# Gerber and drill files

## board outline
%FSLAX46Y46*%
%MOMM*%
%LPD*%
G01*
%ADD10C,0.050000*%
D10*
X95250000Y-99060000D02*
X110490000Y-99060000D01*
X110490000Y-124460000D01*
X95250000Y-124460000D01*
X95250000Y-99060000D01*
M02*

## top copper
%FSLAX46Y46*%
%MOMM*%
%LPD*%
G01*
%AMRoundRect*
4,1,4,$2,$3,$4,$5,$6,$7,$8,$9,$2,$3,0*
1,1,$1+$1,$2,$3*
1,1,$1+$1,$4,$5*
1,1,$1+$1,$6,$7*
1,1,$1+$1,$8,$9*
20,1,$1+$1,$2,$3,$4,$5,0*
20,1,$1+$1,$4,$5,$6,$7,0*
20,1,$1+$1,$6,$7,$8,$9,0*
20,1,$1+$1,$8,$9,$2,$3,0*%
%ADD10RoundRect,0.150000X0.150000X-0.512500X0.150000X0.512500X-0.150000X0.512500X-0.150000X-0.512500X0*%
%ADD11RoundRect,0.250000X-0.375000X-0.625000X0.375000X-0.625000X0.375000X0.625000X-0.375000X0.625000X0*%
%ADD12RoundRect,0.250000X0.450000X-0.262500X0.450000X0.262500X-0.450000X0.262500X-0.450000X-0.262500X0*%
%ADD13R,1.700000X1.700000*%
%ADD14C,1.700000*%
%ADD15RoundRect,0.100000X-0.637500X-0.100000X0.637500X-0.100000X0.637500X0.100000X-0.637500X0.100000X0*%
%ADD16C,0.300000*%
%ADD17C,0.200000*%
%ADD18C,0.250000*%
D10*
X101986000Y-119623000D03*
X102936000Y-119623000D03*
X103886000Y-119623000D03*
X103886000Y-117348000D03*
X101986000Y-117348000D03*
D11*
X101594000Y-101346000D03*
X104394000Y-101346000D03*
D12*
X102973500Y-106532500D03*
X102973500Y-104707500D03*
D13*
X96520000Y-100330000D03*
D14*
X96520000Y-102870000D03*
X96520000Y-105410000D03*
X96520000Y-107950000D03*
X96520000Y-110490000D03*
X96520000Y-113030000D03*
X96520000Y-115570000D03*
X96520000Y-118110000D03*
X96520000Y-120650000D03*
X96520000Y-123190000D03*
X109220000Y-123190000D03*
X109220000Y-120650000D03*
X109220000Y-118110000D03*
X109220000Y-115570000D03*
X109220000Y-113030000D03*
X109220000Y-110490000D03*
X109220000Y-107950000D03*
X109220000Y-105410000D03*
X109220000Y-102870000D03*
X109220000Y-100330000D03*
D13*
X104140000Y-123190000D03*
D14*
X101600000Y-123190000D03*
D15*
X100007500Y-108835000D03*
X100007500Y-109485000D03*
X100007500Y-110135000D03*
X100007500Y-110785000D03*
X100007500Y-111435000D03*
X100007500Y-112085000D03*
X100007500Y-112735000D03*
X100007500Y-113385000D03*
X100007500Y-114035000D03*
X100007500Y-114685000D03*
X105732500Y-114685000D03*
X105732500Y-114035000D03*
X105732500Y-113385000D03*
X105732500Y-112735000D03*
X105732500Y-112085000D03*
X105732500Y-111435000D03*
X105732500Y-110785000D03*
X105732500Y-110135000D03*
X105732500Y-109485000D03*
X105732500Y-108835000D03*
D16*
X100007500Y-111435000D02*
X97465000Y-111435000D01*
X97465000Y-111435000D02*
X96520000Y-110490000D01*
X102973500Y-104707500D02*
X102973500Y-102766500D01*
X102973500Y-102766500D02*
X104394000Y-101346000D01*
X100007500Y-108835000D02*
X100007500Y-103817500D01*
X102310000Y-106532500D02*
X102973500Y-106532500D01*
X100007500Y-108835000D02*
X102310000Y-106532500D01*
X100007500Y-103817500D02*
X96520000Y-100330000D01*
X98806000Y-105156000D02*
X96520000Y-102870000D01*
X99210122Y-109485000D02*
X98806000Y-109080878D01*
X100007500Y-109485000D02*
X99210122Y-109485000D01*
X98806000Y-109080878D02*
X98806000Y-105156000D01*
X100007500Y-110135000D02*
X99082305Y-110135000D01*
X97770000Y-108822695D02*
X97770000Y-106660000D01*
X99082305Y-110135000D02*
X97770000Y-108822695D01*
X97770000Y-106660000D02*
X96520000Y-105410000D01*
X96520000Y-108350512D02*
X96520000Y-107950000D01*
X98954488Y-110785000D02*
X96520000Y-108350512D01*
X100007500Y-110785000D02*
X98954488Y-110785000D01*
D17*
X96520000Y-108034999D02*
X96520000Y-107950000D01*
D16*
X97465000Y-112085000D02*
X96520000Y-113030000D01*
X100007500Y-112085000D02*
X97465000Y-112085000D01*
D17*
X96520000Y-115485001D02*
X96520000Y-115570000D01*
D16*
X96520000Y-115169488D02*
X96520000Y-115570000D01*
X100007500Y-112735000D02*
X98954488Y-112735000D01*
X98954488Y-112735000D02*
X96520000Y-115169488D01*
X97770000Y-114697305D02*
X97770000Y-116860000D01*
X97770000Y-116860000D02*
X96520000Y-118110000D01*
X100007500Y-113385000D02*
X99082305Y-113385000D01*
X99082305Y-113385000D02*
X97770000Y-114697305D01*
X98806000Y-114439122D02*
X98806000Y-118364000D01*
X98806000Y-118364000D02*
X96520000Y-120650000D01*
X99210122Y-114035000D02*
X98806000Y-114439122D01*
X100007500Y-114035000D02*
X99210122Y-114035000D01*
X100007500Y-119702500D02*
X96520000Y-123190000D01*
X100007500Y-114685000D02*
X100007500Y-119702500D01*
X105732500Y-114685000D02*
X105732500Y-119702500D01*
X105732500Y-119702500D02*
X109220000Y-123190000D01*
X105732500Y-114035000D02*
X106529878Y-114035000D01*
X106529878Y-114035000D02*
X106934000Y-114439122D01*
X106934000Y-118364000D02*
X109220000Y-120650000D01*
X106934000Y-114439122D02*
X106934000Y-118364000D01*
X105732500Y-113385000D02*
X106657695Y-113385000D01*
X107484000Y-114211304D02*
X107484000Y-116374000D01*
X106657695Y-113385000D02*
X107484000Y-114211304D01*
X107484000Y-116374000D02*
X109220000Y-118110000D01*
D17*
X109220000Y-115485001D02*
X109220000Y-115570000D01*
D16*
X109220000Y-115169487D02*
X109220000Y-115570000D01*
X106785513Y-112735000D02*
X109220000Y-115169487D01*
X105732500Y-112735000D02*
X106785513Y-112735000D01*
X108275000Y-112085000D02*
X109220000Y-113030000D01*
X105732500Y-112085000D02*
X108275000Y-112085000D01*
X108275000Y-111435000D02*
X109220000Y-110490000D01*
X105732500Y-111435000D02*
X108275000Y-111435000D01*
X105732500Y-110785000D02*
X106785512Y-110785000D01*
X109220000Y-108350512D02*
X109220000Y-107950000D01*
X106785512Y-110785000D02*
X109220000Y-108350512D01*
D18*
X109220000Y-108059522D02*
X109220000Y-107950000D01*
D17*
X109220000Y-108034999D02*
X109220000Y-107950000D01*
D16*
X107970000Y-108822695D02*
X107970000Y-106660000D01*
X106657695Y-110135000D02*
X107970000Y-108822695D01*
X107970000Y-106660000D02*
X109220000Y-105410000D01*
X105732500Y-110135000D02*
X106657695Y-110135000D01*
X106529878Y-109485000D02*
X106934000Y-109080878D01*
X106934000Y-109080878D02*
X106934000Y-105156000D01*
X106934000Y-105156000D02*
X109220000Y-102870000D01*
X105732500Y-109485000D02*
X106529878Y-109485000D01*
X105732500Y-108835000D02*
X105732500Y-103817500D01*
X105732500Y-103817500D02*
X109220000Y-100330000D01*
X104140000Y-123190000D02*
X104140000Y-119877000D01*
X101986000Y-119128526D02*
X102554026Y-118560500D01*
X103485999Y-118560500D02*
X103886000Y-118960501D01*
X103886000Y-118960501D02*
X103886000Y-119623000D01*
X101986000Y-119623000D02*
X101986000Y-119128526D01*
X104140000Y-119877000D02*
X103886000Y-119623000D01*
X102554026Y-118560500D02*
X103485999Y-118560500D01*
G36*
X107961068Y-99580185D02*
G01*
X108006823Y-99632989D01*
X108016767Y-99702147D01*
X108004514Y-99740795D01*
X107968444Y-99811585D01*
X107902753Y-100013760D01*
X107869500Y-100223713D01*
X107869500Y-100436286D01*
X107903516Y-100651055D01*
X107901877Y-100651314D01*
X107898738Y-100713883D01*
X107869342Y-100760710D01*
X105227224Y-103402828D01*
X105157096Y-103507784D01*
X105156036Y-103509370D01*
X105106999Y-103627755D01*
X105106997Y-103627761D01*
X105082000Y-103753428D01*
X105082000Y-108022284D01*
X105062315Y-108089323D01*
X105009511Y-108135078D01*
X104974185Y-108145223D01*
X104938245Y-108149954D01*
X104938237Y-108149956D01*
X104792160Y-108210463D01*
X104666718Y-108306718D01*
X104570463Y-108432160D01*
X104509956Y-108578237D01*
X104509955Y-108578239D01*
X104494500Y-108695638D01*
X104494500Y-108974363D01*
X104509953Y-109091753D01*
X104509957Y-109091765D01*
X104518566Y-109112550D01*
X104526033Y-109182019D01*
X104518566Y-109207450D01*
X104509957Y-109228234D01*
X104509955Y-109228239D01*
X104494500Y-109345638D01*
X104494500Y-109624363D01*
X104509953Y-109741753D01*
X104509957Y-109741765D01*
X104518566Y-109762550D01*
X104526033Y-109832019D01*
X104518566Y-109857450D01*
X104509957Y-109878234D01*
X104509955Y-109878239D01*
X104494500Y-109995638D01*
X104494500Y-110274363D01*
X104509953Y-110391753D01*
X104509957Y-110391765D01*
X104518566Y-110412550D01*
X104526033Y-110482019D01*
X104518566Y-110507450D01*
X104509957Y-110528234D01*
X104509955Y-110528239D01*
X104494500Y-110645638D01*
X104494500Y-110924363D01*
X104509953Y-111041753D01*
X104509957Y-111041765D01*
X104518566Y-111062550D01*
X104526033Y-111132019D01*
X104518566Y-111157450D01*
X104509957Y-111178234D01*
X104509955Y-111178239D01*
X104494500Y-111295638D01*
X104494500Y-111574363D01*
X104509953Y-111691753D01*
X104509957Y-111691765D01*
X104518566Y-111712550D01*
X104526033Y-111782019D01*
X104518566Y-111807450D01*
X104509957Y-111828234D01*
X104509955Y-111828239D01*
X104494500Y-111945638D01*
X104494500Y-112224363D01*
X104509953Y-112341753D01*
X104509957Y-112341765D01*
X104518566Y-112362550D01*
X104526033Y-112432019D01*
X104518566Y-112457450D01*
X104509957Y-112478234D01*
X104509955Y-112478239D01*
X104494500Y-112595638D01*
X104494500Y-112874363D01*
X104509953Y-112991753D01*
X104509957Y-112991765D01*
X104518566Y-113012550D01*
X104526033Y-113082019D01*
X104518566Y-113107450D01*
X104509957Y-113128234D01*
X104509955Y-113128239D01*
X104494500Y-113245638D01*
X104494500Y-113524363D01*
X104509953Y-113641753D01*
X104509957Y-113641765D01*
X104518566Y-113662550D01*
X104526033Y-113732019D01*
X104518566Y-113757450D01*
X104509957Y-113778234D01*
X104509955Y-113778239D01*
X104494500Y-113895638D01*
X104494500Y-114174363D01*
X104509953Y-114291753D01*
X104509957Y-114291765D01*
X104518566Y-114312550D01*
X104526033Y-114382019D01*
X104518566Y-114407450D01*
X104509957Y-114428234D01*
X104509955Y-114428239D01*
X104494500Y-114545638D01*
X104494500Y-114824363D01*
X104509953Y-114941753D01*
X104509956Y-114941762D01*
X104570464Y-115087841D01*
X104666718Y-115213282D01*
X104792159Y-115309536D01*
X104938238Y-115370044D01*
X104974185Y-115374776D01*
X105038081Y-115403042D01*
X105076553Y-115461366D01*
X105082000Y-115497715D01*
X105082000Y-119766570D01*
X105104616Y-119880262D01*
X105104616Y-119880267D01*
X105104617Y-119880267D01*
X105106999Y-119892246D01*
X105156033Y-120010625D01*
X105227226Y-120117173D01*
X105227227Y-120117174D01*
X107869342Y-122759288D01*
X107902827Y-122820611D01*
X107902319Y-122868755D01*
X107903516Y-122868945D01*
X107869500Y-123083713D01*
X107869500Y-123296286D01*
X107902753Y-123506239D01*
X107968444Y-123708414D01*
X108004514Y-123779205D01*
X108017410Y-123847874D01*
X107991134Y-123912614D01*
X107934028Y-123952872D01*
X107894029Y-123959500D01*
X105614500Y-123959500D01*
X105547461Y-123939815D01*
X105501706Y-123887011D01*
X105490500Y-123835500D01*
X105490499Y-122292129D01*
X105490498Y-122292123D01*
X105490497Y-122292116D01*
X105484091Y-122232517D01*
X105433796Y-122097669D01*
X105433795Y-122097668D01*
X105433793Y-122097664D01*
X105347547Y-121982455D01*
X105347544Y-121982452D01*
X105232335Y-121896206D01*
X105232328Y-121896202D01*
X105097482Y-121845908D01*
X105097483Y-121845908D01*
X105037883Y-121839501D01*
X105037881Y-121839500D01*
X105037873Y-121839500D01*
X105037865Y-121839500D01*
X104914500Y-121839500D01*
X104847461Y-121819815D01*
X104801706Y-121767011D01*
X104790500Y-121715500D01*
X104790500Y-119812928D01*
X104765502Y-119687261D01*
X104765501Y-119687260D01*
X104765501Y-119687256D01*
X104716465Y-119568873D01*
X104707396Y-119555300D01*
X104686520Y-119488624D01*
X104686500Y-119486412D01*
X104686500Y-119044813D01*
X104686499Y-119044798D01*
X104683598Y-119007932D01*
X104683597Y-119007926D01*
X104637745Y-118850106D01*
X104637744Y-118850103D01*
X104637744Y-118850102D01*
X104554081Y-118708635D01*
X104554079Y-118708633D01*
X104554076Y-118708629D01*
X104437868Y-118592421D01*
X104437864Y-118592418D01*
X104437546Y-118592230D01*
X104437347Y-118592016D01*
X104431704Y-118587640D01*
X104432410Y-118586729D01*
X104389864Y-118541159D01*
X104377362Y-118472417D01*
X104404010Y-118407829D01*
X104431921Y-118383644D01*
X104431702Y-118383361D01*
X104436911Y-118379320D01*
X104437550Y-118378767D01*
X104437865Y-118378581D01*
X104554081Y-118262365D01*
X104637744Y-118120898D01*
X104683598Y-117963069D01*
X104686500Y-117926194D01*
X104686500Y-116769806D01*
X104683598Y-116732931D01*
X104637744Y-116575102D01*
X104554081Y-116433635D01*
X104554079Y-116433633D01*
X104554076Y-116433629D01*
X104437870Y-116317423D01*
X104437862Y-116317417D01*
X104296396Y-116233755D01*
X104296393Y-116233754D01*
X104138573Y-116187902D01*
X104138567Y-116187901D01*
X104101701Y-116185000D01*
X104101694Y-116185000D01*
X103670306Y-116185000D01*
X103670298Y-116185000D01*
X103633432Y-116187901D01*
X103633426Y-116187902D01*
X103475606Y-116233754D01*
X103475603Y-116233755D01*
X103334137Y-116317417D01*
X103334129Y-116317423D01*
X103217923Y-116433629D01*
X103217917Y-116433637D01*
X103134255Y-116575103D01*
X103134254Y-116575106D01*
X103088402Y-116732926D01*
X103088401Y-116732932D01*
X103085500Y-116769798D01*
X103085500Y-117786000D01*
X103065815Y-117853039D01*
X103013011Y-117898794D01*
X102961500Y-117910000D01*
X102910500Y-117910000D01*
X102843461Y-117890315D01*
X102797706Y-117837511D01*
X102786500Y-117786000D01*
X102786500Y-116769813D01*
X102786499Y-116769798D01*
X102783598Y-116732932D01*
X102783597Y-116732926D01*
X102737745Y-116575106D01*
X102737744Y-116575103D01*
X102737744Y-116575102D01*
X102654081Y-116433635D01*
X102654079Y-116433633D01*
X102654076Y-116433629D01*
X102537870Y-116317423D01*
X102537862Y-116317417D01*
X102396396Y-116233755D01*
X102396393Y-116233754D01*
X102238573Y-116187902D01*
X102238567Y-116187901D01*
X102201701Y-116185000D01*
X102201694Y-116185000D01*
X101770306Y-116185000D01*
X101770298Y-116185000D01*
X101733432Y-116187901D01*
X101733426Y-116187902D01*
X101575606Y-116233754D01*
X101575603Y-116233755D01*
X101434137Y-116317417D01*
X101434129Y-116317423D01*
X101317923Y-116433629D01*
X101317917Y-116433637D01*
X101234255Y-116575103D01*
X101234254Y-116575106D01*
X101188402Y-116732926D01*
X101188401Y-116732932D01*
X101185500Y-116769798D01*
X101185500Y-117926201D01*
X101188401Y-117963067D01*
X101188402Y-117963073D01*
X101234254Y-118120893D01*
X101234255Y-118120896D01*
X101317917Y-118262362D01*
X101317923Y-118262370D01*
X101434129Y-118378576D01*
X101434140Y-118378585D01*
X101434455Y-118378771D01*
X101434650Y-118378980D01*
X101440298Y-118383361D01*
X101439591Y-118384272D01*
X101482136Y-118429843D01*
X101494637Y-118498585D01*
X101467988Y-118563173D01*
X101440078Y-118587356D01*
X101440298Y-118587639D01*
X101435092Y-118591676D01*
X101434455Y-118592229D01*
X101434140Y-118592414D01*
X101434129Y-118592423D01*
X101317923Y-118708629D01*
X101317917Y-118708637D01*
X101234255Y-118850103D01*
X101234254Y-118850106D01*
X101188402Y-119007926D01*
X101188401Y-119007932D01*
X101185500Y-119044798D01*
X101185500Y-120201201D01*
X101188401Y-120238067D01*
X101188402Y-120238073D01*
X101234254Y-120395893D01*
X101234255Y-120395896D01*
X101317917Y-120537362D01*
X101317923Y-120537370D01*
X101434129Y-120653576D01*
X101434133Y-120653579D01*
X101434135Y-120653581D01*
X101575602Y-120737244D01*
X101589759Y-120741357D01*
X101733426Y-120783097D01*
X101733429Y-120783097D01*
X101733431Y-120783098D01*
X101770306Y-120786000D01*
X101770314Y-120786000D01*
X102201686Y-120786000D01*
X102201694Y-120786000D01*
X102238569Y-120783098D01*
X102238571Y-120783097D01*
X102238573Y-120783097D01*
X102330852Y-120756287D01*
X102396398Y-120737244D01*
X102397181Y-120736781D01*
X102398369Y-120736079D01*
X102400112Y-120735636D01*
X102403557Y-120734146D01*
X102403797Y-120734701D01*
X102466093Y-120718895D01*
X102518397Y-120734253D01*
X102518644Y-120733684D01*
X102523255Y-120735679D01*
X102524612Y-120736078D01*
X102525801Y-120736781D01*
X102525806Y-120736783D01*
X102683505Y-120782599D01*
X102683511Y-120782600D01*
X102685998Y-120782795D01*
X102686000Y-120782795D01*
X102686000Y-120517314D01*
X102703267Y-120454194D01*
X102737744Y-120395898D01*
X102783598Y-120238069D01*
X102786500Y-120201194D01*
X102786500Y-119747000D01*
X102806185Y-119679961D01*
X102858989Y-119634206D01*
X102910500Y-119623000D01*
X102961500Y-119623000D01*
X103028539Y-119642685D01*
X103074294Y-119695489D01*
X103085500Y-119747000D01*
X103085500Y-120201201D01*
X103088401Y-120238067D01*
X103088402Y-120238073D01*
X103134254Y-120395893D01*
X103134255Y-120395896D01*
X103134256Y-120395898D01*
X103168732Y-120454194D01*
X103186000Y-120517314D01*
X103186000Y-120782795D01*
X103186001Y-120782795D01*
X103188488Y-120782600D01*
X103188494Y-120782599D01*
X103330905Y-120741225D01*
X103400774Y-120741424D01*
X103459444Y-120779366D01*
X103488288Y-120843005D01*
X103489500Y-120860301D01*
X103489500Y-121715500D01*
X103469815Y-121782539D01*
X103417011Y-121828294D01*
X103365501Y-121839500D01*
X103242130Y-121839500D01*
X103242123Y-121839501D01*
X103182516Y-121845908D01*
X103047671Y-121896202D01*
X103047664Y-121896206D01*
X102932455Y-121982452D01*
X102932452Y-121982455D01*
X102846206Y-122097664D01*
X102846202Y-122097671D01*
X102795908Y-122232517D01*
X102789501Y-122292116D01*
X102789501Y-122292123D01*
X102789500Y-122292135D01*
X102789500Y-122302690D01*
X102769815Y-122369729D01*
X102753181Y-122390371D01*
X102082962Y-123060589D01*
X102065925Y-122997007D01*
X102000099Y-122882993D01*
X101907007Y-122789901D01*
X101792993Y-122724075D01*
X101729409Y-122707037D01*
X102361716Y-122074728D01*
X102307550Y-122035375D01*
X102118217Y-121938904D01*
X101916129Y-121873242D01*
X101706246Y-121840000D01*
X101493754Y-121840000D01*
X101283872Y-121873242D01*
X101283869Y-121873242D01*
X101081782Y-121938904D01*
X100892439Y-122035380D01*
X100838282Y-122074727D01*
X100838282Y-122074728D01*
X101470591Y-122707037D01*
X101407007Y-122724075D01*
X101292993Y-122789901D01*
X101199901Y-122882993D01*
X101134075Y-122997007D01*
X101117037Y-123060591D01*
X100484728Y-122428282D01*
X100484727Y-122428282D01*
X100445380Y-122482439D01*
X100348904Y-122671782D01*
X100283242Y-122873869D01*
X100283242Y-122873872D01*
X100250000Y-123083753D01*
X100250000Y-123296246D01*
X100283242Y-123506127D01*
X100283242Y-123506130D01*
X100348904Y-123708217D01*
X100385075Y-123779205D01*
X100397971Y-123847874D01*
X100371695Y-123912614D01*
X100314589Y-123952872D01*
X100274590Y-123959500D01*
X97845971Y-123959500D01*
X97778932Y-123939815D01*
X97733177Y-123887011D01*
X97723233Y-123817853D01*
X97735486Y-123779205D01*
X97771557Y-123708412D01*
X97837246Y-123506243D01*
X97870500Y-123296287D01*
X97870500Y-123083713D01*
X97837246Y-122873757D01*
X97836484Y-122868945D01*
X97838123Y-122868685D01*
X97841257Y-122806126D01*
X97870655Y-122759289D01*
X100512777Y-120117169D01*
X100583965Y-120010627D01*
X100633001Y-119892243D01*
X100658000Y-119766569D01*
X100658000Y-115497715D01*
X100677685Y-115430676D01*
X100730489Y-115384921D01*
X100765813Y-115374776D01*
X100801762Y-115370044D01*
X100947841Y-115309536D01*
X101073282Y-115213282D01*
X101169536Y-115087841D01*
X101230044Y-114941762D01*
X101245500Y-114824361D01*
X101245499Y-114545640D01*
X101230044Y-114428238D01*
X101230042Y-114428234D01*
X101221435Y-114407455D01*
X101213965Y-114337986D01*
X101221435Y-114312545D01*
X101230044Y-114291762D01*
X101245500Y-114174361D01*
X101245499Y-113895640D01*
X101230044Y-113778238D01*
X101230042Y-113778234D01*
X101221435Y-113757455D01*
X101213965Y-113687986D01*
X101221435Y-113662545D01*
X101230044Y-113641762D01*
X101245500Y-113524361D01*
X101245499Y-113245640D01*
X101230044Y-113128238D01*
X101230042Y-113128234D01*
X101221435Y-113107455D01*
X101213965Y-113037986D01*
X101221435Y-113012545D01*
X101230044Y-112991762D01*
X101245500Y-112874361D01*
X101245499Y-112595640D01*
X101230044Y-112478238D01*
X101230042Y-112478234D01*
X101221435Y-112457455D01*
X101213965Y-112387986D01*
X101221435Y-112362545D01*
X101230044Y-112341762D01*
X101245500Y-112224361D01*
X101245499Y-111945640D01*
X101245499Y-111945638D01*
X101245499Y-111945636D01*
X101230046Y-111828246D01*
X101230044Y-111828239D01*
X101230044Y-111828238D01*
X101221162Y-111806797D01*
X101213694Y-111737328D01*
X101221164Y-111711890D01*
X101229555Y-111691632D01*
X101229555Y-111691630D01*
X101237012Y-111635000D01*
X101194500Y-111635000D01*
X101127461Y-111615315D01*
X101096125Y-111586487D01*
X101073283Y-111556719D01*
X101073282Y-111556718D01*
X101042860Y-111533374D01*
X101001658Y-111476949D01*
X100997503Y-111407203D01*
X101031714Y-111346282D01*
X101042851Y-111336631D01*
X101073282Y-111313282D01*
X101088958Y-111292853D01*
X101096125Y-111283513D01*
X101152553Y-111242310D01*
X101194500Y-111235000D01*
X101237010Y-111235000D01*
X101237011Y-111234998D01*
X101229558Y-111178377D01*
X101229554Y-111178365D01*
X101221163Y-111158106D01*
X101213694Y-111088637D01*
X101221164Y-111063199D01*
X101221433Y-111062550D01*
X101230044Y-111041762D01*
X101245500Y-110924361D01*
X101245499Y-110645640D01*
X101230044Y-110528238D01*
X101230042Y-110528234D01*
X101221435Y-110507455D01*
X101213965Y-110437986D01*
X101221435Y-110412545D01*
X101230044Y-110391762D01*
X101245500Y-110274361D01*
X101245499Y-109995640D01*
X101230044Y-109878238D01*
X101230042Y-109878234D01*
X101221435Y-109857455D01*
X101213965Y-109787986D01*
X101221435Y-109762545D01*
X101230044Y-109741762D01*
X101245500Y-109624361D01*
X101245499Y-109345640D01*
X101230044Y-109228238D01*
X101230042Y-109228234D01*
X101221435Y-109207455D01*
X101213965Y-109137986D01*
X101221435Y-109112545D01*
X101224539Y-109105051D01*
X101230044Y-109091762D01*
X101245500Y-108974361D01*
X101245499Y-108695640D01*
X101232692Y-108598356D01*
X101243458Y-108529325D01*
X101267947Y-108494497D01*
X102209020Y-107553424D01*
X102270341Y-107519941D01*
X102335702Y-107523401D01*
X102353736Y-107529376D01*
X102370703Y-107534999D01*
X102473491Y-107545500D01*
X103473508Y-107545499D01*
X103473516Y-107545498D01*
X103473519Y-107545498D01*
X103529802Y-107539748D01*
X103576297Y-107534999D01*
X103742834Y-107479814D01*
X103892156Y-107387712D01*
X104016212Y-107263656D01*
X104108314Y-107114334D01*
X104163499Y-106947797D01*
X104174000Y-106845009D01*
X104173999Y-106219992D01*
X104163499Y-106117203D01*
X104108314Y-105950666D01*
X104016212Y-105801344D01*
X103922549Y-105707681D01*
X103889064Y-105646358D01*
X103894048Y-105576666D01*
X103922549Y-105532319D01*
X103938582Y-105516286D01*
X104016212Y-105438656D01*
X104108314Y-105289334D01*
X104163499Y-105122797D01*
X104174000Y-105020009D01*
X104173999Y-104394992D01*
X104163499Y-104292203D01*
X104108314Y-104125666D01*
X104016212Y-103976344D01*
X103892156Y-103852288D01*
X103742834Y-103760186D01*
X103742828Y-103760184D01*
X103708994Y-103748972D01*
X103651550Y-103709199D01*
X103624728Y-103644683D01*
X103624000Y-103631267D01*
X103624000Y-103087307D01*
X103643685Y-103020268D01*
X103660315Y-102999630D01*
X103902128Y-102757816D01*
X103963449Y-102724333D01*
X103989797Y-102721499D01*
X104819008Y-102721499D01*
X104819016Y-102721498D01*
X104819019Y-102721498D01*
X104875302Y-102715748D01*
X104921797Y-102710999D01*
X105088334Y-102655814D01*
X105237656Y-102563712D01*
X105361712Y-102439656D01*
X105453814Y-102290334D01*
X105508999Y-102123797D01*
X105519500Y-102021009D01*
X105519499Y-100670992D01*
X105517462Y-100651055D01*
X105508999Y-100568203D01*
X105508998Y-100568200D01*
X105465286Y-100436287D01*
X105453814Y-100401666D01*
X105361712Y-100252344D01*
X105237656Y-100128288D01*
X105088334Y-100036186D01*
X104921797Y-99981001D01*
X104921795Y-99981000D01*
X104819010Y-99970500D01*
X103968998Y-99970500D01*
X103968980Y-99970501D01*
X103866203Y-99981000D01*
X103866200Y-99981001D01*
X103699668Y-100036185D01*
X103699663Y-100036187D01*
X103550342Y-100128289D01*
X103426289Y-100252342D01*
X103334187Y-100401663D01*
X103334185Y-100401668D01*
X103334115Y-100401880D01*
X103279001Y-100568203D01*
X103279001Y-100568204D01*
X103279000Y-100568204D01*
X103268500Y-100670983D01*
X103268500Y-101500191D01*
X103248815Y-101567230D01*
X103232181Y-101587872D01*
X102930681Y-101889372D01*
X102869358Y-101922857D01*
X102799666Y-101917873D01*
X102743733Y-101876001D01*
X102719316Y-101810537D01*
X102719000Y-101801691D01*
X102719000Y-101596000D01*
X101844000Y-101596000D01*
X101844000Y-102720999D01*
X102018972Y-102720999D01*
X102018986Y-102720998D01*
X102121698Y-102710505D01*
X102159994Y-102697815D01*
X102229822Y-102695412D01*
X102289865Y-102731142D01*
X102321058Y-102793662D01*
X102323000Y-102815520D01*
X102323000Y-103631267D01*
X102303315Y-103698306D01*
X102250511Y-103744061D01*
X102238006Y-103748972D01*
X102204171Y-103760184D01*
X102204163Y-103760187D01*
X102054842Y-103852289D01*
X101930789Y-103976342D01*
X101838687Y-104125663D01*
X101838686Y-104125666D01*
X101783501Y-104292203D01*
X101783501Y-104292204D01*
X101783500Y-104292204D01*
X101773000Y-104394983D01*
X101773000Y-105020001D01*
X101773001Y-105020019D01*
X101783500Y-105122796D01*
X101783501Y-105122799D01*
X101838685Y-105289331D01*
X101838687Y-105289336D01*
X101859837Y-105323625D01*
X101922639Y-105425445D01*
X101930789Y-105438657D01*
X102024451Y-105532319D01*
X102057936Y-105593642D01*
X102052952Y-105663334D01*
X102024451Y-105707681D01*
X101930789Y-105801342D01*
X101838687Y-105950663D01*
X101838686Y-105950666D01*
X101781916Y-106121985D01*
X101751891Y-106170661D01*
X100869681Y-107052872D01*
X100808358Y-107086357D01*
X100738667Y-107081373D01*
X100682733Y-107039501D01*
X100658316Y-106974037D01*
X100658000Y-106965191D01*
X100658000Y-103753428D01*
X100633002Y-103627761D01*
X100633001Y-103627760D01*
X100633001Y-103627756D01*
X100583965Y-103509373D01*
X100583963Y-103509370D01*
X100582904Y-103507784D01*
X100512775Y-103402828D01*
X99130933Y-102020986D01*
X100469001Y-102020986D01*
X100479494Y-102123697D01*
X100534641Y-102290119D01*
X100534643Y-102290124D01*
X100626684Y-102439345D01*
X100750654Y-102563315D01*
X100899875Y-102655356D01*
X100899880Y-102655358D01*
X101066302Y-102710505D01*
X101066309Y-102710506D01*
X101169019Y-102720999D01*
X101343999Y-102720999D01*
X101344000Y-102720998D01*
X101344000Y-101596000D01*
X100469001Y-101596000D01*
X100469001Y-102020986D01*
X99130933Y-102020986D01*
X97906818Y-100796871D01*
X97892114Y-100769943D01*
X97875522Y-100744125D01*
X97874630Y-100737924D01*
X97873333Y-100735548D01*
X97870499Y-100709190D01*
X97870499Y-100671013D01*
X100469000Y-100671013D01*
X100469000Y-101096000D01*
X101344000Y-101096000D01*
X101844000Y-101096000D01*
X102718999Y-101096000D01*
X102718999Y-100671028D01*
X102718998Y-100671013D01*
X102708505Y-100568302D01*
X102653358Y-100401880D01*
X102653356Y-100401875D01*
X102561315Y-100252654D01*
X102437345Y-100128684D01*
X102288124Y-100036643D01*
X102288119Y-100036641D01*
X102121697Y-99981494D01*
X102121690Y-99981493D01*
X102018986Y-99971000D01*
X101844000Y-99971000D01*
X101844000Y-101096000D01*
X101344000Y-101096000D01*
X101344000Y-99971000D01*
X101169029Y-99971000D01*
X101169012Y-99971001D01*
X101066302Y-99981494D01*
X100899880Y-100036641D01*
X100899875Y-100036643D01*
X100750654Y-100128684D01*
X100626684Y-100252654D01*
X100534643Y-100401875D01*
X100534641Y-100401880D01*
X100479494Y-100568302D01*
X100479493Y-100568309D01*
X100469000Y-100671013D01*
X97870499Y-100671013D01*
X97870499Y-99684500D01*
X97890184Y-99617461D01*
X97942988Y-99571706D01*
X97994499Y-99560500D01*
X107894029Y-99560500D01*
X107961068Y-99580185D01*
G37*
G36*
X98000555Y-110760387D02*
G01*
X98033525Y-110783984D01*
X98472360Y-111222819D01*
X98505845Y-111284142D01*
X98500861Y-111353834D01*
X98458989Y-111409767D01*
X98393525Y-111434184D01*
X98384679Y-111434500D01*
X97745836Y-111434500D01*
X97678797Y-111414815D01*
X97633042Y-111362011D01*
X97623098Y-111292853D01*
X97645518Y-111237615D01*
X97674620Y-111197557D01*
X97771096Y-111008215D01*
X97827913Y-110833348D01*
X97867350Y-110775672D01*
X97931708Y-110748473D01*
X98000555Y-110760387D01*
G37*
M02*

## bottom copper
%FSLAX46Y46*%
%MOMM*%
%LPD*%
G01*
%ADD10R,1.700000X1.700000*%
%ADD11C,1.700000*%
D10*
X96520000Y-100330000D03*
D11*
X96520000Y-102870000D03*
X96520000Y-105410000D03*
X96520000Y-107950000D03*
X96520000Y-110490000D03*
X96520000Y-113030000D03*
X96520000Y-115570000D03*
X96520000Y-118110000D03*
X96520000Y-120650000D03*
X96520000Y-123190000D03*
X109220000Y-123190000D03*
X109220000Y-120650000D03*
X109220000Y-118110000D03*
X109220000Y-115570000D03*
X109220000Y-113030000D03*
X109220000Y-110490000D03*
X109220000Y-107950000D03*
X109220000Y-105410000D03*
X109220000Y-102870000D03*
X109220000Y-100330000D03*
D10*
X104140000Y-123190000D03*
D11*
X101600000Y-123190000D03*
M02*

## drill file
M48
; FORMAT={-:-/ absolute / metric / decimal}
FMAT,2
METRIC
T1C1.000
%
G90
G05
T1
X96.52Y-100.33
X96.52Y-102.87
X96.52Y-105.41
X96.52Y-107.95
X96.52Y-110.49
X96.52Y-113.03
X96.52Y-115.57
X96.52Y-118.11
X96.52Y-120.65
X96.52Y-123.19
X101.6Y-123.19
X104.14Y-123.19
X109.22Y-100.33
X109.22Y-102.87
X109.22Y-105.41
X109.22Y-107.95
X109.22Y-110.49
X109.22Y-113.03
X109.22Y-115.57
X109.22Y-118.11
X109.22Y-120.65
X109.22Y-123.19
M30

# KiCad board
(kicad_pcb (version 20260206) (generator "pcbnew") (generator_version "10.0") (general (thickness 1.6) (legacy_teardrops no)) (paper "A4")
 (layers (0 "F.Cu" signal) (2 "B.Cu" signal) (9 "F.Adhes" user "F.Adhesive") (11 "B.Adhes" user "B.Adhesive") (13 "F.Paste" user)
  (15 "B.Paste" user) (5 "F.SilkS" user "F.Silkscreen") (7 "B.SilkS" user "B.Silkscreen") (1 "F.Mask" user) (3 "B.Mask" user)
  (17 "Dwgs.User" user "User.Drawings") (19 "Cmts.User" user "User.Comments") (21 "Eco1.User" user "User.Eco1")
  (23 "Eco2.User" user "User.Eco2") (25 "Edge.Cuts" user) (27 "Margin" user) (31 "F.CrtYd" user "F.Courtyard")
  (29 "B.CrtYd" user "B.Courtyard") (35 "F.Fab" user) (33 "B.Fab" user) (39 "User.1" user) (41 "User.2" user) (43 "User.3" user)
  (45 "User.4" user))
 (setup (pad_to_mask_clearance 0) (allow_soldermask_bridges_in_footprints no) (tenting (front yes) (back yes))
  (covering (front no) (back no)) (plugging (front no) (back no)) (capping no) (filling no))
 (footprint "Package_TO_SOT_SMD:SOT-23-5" (layer "F.Cu") (at 102.936 118.4855 90)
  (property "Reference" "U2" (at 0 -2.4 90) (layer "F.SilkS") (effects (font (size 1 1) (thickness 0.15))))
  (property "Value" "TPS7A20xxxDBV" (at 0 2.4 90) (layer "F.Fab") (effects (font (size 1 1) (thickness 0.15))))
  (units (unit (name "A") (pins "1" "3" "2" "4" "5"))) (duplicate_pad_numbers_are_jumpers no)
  (pad "1" smd roundrect (at -1.1375 -0.95 90) (size 1.325 0.6) (layers "F.Cu" "F.Mask" "F.Paste") (roundrect_rratio 0.25)
   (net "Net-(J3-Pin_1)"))
  (pad "2" smd roundrect (at -1.1375 0 90) (size 1.325 0.6) (layers "F.Cu" "F.Mask" "F.Paste") (roundrect_rratio 0.25) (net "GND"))
  (pad "3" smd roundrect (at -1.1375 0.95 90) (size 1.325 0.6) (layers "F.Cu" "F.Mask" "F.Paste") (roundrect_rratio 0.25)
   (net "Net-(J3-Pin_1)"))
  (pad "4" smd roundrect (at 1.1375 0.95 90) (size 1.325 0.6) (layers "F.Cu" "F.Mask" "F.Paste") (roundrect_rratio 0.25)
   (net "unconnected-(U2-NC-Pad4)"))
  (pad "5" smd roundrect (at 1.1375 -0.95 90) (size 1.325 0.6) (layers "F.Cu" "F.Mask" "F.Paste") (roundrect_rratio 0.25)
   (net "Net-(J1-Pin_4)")))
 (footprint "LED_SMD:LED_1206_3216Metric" (layer "F.Cu") (at 102.994 101.346)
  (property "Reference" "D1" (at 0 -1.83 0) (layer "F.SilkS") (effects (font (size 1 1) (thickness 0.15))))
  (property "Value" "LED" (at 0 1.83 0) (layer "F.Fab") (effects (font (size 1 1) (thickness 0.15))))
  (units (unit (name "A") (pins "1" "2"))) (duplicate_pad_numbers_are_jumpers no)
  (pad "1" smd roundrect (at -1.4 0) (size 1.25 1.75) (layers "F.Cu" "F.Mask" "F.Paste") (roundrect_rratio 0.2) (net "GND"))
  (pad "2" smd roundrect (at 1.4 0) (size 1.25 1.75) (layers "F.Cu" "F.Mask" "F.Paste") (roundrect_rratio 0.2) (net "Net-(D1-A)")))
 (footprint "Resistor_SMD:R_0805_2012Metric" (layer "F.Cu") (at 102.9735 105.62 90)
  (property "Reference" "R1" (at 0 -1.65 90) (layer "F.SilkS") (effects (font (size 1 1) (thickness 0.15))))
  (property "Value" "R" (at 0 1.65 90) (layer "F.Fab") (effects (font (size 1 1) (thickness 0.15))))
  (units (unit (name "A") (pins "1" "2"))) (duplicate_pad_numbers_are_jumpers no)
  (pad "1" smd roundrect (at -0.9125 0 90) (size 1.025 1.4) (layers "F.Cu" "F.Mask" "F.Paste") (roundrect_rratio 0.243902)
   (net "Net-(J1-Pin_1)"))
  (pad "2" smd roundrect (at 0.9125 0 90) (size 1.025 1.4) (layers "F.Cu" "F.Mask" "F.Paste") (roundrect_rratio 0.243902) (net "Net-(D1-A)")))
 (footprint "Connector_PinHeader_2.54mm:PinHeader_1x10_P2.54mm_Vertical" (layer "F.Cu") (at 96.52 100.33)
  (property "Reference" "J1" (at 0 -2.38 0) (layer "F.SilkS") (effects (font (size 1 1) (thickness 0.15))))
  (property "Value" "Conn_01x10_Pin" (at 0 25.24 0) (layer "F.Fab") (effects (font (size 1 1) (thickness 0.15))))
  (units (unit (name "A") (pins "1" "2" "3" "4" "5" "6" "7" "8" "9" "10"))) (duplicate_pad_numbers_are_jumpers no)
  (pad "1" thru_hole rect (at 0 0) (size 1.7 1.7) (drill 1) (layers "*.Cu" "*.Mask") (remove_unused_layers no) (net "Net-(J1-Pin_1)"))
  (pad "2" thru_hole circle (at 0 2.54) (size 1.7 1.7) (drill 1) (layers "*.Cu" "*.Mask") (remove_unused_layers no) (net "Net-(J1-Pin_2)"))
  (pad "3" thru_hole circle (at 0 5.08) (size 1.7 1.7) (drill 1) (layers "*.Cu" "*.Mask") (remove_unused_layers no) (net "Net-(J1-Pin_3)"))
  (pad "4" thru_hole circle (at 0 7.62) (size 1.7 1.7) (drill 1) (layers "*.Cu" "*.Mask") (remove_unused_layers no) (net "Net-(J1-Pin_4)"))
  (pad "5" thru_hole circle (at 0 10.16) (size 1.7 1.7) (drill 1) (layers "*.Cu" "*.Mask") (remove_unused_layers no) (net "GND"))
  (pad "6" thru_hole circle (at 0 12.7) (size 1.7 1.7) (drill 1) (layers "*.Cu" "*.Mask") (remove_unused_layers no) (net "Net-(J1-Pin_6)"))
  (pad "7" thru_hole circle (at 0 15.24) (size 1.7 1.7) (drill 1) (layers "*.Cu" "*.Mask") (remove_unused_layers no) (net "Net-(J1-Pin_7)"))
  (pad "8" thru_hole circle (at 0 17.78) (size 1.7 1.7) (drill 1) (layers "*.Cu" "*.Mask") (remove_unused_layers no) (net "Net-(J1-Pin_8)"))
  (pad "9" thru_hole circle (at 0 20.32) (size 1.7 1.7) (drill 1) (layers "*.Cu" "*.Mask") (remove_unused_layers no) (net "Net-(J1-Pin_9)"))
  (pad "10" thru_hole circle (at 0 22.86) (size 1.7 1.7) (drill 1) (layers "*.Cu" "*.Mask") (remove_unused_layers no)
   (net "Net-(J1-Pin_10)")))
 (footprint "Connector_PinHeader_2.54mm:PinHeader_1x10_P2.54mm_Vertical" (layer "F.Cu") (at 109.22 123.19 180)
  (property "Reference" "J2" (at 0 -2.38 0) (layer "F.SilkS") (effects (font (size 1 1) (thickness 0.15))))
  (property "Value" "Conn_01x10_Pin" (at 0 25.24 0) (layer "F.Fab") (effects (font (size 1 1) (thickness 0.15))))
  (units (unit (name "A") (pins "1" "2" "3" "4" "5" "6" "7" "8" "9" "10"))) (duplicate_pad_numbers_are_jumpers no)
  (pad "1" thru_hole circle (at 0 0 180) (size 1.7 1.7) (drill 1) (layers "*.Cu" "*.Mask") (remove_unused_layers no) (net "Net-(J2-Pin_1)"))
  (pad "2" thru_hole circle (at 0 2.54 180) (size 1.7 1.7) (drill 1) (layers "*.Cu" "*.Mask") (remove_unused_layers no)
   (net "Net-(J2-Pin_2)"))
  (pad "3" thru_hole circle (at 0 5.08 180) (size 1.7 1.7) (drill 1) (layers "*.Cu" "*.Mask") (remove_unused_layers no)
   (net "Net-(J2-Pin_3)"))
  (pad "4" thru_hole circle (at 0 7.62 180) (size 1.7 1.7) (drill 1) (layers "*.Cu" "*.Mask") (remove_unused_layers no)
   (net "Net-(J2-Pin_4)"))
  (pad "5" thru_hole circle (at 0 10.16 180) (size 1.7 1.7) (drill 1) (layers "*.Cu" "*.Mask") (remove_unused_layers no)
   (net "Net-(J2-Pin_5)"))
  (pad "6" thru_hole circle (at 0 12.7 180) (size 1.7 1.7) (drill 1) (layers "*.Cu" "*.Mask") (remove_unused_layers no)
   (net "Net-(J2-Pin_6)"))
  (pad "7" thru_hole circle (at 0 15.24 180) (size 1.7 1.7) (drill 1) (layers "*.Cu" "*.Mask") (remove_unused_layers no)
   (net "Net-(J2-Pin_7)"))
  (pad "8" thru_hole circle (at 0 17.78 180) (size 1.7 1.7) (drill 1) (layers "*.Cu" "*.Mask") (remove_unused_layers no)
   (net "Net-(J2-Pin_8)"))
  (pad "9" thru_hole circle (at 0 20.32 180) (size 1.7 1.7) (drill 1) (layers "*.Cu" "*.Mask") (remove_unused_layers no)
   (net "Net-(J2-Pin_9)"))
  (pad "10" thru_hole circle (at 0 22.86 180) (size 1.7 1.7) (drill 1) (layers "*.Cu" "*.Mask") (remove_unused_layers no)
   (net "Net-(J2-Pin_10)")))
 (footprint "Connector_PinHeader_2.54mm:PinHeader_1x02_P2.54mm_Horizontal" (layer "F.Cu") (at 104.14 123.19 -90)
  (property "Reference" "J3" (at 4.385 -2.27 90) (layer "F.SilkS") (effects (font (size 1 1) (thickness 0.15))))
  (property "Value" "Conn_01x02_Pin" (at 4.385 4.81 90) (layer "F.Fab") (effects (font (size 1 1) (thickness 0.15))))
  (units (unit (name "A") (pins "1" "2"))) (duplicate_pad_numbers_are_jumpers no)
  (pad "1" thru_hole rect (at 0 0 270) (size 1.7 1.7) (drill 1) (layers "*.Cu" "*.Mask") (remove_unused_layers no) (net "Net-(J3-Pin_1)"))
  (pad "2" thru_hole circle (at 0 2.54 270) (size 1.7 1.7) (drill 1) (layers "*.Cu" "*.Mask") (remove_unused_layers no) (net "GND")))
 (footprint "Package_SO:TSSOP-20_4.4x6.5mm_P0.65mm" (layer "F.Cu") (at 102.87 111.76)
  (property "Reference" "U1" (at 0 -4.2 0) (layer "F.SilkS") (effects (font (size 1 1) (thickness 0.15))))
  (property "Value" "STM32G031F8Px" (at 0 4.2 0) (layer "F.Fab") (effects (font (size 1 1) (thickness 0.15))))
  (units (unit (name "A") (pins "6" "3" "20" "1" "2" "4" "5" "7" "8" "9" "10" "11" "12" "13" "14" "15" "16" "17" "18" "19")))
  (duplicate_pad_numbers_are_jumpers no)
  (pad "1" smd roundrect (at -2.8625 -2.925) (size 1.475 0.4) (layers "F.Cu" "F.Mask" "F.Paste") (roundrect_rratio 0.25)
   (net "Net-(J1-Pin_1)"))
  (pad "2" smd roundrect (at -2.8625 -2.275) (size 1.475 0.4) (layers "F.Cu" "F.Mask" "F.Paste") (roundrect_rratio 0.25)
   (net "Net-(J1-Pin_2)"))
  (pad "3" smd roundrect (at -2.8625 -1.625) (size 1.475 0.4) (layers "F.Cu" "F.Mask" "F.Paste") (roundrect_rratio 0.25)
   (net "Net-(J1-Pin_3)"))
  (pad "4" smd roundrect (at -2.8625 -0.975) (size 1.475 0.4) (layers "F.Cu" "F.Mask" "F.Paste") (roundrect_rratio 0.25)
   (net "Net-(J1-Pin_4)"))
  (pad "5" smd roundrect (at -2.8625 -0.325) (size 1.475 0.4) (layers "F.Cu" "F.Mask" "F.Paste") (roundrect_rratio 0.25) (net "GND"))
  (pad "6" smd roundrect (at -2.8625 0.325) (size 1.475 0.4) (layers "F.Cu" "F.Mask" "F.Paste") (roundrect_rratio 0.25)
   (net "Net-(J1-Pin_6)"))
  (pad "7" smd roundrect (at -2.8625 0.975) (size 1.475 0.4) (layers "F.Cu" "F.Mask" "F.Paste") (roundrect_rratio 0.25)
   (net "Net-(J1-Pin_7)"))
  (pad "8" smd roundrect (at -2.8625 1.625) (size 1.475 0.4) (layers "F.Cu" "F.Mask" "F.Paste") (roundrect_rratio 0.25)
   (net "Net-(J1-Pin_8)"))
  (pad "9" smd roundrect (at -2.8625 2.275) (size 1.475 0.4) (layers "F.Cu" "F.Mask" "F.Paste") (roundrect_rratio 0.25)
   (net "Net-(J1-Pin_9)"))
  (pad "10" smd roundrect (at -2.8625 2.925) (size 1.475 0.4) (layers "F.Cu" "F.Mask" "F.Paste") (roundrect_rratio 0.25)
   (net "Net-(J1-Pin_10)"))
  (pad "11" smd roundrect (at 2.8625 2.925) (size 1.475 0.4) (layers "F.Cu" "F.Mask" "F.Paste") (roundrect_rratio 0.25)
   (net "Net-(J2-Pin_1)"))
  (pad "12" smd roundrect (at 2.8625 2.275) (size 1.475 0.4) (layers "F.Cu" "F.Mask" "F.Paste") (roundrect_rratio 0.25)
   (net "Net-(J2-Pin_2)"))
  (pad "13" smd roundrect (at 2.8625 1.625) (size 1.475 0.4) (layers "F.Cu" "F.Mask" "F.Paste") (roundrect_rratio 0.25)
   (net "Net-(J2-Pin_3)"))
  (pad "14" smd roundrect (at 2.8625 0.975) (size 1.475 0.4) (layers "F.Cu" "F.Mask" "F.Paste") (roundrect_rratio 0.25)
   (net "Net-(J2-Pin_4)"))
  (pad "15" smd roundrect (at 2.8625 0.325) (size 1.475 0.4) (layers "F.Cu" "F.Mask" "F.Paste") (roundrect_rratio 0.25)
   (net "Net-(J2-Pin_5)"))
  (pad "16" smd roundrect (at 2.8625 -0.325) (size 1.475 0.4) (layers "F.Cu" "F.Mask" "F.Paste") (roundrect_rratio 0.25)
   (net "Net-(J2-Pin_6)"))
  (pad "17" smd roundrect (at 2.8625 -0.975) (size 1.475 0.4) (layers "F.Cu" "F.Mask" "F.Paste") (roundrect_rratio 0.25)
   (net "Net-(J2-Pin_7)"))
  (pad "18" smd roundrect (at 2.8625 -1.625) (size 1.475 0.4) (layers "F.Cu" "F.Mask" "F.Paste") (roundrect_rratio 0.25)
   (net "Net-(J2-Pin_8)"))
  (pad "19" smd roundrect (at 2.8625 -2.275) (size 1.475 0.4) (layers "F.Cu" "F.Mask" "F.Paste") (roundrect_rratio 0.25)
   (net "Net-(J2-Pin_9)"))
  (pad "20" smd roundrect (at 2.8625 -2.925) (size 1.475 0.4) (layers "F.Cu" "F.Mask" "F.Paste") (roundrect_rratio 0.25)
   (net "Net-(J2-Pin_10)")))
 (gr_rect (start 95.25 99.06) (end 110.49 124.46) (stroke (width 0.05) (type default)) (fill no) (layer "Edge.Cuts"))
 (segment (start 100.0075 111.435) (end 97.465 111.435) (width 0.3) (layer "F.Cu") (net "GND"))
 (segment (start 97.465 111.435) (end 96.52 110.49) (width 0.3) (layer "F.Cu") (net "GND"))
 (segment (start 102.9735 104.7075) (end 102.9735 102.7665) (width 0.3) (layer "F.Cu") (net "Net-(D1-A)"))
 (segment (start 102.9735 102.7665) (end 104.394 101.346) (width 0.3) (layer "F.Cu") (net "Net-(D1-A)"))
 (segment (start 100.0075 108.835) (end 100.0075 103.8175) (width 0.3) (layer "F.Cu") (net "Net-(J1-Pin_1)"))
 (segment (start 102.31 106.5325) (end 102.9735 106.5325) (width 0.3) (layer "F.Cu") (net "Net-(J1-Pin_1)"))
 (segment (start 100.0075 108.835) (end 102.31 106.5325) (width 0.3) (layer "F.Cu") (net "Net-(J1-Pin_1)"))
 (segment (start 100.0075 103.8175) (end 96.52 100.33) (width 0.3) (layer "F.Cu") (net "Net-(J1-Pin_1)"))
 (segment (start 98.806 105.156) (end 96.52 102.87) (width 0.3) (layer "F.Cu") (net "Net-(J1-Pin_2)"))
 (segment (start 99.210122 109.485) (end 98.806 109.080878) (width 0.3) (layer "F.Cu") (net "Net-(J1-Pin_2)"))
 (segment (start 100.0075 109.485) (end 99.210122 109.485) (width 0.3) (layer "F.Cu") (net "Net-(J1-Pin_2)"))
 (segment (start 98.806 109.080878) (end 98.806 105.156) (width 0.3) (layer "F.Cu") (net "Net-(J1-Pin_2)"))
 (segment (start 100.0075 110.135) (end 99.082305 110.135) (width 0.3) (layer "F.Cu") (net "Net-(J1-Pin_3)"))
 (segment (start 97.77 108.822695) (end 97.77 106.66) (width 0.3) (layer "F.Cu") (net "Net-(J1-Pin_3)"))
 (segment (start 99.082305 110.135) (end 97.77 108.822695) (width 0.3) (layer "F.Cu") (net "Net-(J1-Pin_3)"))
 (segment (start 97.77 106.66) (end 96.52 105.41) (width 0.3) (layer "F.Cu") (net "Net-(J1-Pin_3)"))
 (segment (start 96.52 108.350512) (end 96.52 107.95) (width 0.3) (layer "F.Cu") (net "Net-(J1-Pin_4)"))
 (segment (start 98.954488 110.785) (end 96.52 108.350512) (width 0.3) (layer "F.Cu") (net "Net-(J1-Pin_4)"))
 (segment (start 100.0075 110.785) (end 98.954488 110.785) (width 0.3) (layer "F.Cu") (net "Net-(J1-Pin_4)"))
 (segment (start 96.52 108.034999) (end 96.52 107.95) (width 0.2) (layer "F.Cu") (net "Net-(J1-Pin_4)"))
 (segment (start 97.465 112.085) (end 96.52 113.03) (width 0.3) (layer "F.Cu") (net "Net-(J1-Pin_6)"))
 (segment (start 100.0075 112.085) (end 97.465 112.085) (width 0.3) (layer "F.Cu") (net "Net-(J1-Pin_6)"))
 (segment (start 96.52 115.485001) (end 96.52 115.57) (width 0.2) (layer "F.Cu") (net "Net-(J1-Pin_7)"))
 (segment (start 96.52 115.169488) (end 96.52 115.57) (width 0.3) (layer "F.Cu") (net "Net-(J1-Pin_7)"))
 (segment (start 100.0075 112.735) (end 98.954488 112.735) (width 0.3) (layer "F.Cu") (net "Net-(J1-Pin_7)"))
 (segment (start 98.954488 112.735) (end 96.52 115.169488) (width 0.3) (layer "F.Cu") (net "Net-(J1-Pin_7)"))
 (segment (start 97.77 114.697305) (end 97.77 116.86) (width 0.3) (layer "F.Cu") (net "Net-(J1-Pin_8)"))
 (segment (start 97.77 116.86) (end 96.52 118.11) (width 0.3) (layer "F.Cu") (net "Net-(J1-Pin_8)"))
 (segment (start 100.0075 113.385) (end 99.082305 113.385) (width 0.3) (layer "F.Cu") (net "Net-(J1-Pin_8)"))
 (segment (start 99.082305 113.385) (end 97.77 114.697305) (width 0.3) (layer "F.Cu") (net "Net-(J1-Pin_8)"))
 (segment (start 98.806 114.439122) (end 98.806 118.364) (width 0.3) (layer "F.Cu") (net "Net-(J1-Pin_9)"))
 (segment (start 98.806 118.364) (end 96.52 120.65) (width 0.3) (layer "F.Cu") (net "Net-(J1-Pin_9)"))
 (segment (start 99.210122 114.035) (end 98.806 114.439122) (width 0.3) (layer "F.Cu") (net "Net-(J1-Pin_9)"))
 (segment (start 100.0075 114.035) (end 99.210122 114.035) (width 0.3) (layer "F.Cu") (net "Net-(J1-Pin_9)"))
 (segment (start 100.0075 119.7025) (end 96.52 123.19) (width 0.3) (layer "F.Cu") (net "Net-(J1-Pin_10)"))
 (segment (start 100.0075 114.685) (end 100.0075 119.7025) (width 0.3) (layer "F.Cu") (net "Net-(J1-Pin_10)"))
 (segment (start 105.7325 114.685) (end 105.7325 119.7025) (width 0.3) (layer "F.Cu") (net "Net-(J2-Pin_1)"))
 (segment (start 105.7325 119.7025) (end 109.22 123.19) (width 0.3) (layer "F.Cu") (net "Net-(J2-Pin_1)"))
 (segment (start 105.7325 114.035) (end 106.529878 114.035) (width 0.3) (layer "F.Cu") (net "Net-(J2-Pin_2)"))
 (segment (start 106.529878 114.035) (end 106.934 114.439122) (width 0.3) (layer "F.Cu") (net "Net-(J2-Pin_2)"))
 (segment (start 106.934 118.364) (end 109.22 120.65) (width 0.3) (layer "F.Cu") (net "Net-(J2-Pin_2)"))
 (segment (start 106.934 114.439122) (end 106.934 118.364) (width 0.3) (layer "F.Cu") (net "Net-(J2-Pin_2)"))
 (segment (start 105.7325 113.385) (end 106.657695 113.385) (width 0.3) (layer "F.Cu") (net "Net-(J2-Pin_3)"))
 (segment (start 107.484 114.211304) (end 107.484 116.374) (width 0.3) (layer "F.Cu") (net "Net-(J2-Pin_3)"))
 (segment (start 106.657695 113.385) (end 107.484 114.211304) (width 0.3) (layer "F.Cu") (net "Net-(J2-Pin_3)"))
 (segment (start 107.484 116.374) (end 109.22 118.11) (width 0.3) (layer "F.Cu") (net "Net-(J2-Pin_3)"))
 (segment (start 109.22 115.485001) (end 109.22 115.57) (width 0.2) (layer "F.Cu") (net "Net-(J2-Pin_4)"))
 (segment (start 109.22 115.169487) (end 109.22 115.57) (width 0.3) (layer "F.Cu") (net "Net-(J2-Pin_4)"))
 (segment (start 106.785513 112.735) (end 109.22 115.169487) (width 0.3) (layer "F.Cu") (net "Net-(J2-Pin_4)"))
 (segment (start 105.7325 112.735) (end 106.785513 112.735) (width 0.3) (layer "F.Cu") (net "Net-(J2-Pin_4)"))
 (segment (start 108.275 112.085) (end 109.22 113.03) (width 0.3) (layer "F.Cu") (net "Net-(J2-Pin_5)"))
 (segment (start 105.7325 112.085) (end 108.275 112.085) (width 0.3) (layer "F.Cu") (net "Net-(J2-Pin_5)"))
 (segment (start 108.275 111.435) (end 109.22 110.49) (width 0.3) (layer "F.Cu") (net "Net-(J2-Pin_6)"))
 (segment (start 105.7325 111.435) (end 108.275 111.435) (width 0.3) (layer "F.Cu") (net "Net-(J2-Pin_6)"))
 (segment (start 105.7325 110.785) (end 106.785512 110.785) (width 0.3) (layer "F.Cu") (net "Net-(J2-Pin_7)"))
 (segment (start 109.22 108.350512) (end 109.22 107.95) (width 0.3) (layer "F.Cu") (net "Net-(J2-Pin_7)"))
 (segment (start 106.785512 110.785) (end 109.22 108.350512) (width 0.3) (layer "F.Cu") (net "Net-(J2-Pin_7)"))
 (segment (start 109.22 108.059522) (end 109.22 107.95) (width 0.25) (layer "F.Cu") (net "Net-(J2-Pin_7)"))
 (segment (start 109.22 108.034999) (end 109.22 107.95) (width 0.2) (layer "F.Cu") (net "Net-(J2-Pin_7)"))
 (segment (start 107.97 108.822695) (end 107.97 106.66) (width 0.3) (layer "F.Cu") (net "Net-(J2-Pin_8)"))
 (segment (start 106.657695 110.135) (end 107.97 108.822695) (width 0.3) (layer "F.Cu") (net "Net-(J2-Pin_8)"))
 (segment (start 107.97 106.66) (end 109.22 105.41) (width 0.3) (layer "F.Cu") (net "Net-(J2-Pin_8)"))
 (segment (start 105.7325 110.135) (end 106.657695 110.135) (width 0.3) (layer "F.Cu") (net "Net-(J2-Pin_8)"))
 (segment (start 106.529878 109.485) (end 106.934 109.080878) (width 0.3) (layer "F.Cu") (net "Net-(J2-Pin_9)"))
 (segment (start 106.934 109.080878) (end 106.934 105.156) (width 0.3) (layer "F.Cu") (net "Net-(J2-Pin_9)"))
 (segment (start 106.934 105.156) (end 109.22 102.87) (width 0.3) (layer "F.Cu") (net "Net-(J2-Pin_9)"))
 (segment (start 105.7325 109.485) (end 106.529878 109.485) (width 0.3) (layer "F.Cu") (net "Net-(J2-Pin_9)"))
 (segment (start 105.7325 108.835) (end 105.7325 103.8175) (width 0.3) (layer "F.Cu") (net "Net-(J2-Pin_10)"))
 (segment (start 105.7325 103.8175) (end 109.22 100.33) (width 0.3) (layer "F.Cu") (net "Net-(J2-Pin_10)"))
 (segment (start 104.14 123.19) (end 104.14 119.877) (width 0.3) (layer "F.Cu") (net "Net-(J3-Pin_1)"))
 (segment (start 101.986 119.128526) (end 102.554026 118.5605) (width 0.3) (layer "F.Cu") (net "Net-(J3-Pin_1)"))
 (segment (start 103.485999 118.5605) (end 103.886 118.960501) (width 0.3) (layer "F.Cu") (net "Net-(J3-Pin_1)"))
 (segment (start 103.886 118.960501) (end 103.886 119.623) (width 0.3) (layer "F.Cu") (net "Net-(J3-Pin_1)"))
 (segment (start 101.986 119.623) (end 101.986 119.128526) (width 0.3) (layer "F.Cu") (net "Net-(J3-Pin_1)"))
 (segment (start 104.14 119.877) (end 103.886 119.623) (width 0.3) (layer "F.Cu") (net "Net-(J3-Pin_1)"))
 (segment (start 102.554026 118.5605) (end 103.485999 118.5605) (width 0.3) (layer "F.Cu") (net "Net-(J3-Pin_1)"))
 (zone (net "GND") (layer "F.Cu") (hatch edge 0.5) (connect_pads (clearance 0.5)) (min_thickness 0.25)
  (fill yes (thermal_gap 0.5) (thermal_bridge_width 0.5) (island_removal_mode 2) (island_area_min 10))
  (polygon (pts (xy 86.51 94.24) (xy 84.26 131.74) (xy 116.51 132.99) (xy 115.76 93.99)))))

